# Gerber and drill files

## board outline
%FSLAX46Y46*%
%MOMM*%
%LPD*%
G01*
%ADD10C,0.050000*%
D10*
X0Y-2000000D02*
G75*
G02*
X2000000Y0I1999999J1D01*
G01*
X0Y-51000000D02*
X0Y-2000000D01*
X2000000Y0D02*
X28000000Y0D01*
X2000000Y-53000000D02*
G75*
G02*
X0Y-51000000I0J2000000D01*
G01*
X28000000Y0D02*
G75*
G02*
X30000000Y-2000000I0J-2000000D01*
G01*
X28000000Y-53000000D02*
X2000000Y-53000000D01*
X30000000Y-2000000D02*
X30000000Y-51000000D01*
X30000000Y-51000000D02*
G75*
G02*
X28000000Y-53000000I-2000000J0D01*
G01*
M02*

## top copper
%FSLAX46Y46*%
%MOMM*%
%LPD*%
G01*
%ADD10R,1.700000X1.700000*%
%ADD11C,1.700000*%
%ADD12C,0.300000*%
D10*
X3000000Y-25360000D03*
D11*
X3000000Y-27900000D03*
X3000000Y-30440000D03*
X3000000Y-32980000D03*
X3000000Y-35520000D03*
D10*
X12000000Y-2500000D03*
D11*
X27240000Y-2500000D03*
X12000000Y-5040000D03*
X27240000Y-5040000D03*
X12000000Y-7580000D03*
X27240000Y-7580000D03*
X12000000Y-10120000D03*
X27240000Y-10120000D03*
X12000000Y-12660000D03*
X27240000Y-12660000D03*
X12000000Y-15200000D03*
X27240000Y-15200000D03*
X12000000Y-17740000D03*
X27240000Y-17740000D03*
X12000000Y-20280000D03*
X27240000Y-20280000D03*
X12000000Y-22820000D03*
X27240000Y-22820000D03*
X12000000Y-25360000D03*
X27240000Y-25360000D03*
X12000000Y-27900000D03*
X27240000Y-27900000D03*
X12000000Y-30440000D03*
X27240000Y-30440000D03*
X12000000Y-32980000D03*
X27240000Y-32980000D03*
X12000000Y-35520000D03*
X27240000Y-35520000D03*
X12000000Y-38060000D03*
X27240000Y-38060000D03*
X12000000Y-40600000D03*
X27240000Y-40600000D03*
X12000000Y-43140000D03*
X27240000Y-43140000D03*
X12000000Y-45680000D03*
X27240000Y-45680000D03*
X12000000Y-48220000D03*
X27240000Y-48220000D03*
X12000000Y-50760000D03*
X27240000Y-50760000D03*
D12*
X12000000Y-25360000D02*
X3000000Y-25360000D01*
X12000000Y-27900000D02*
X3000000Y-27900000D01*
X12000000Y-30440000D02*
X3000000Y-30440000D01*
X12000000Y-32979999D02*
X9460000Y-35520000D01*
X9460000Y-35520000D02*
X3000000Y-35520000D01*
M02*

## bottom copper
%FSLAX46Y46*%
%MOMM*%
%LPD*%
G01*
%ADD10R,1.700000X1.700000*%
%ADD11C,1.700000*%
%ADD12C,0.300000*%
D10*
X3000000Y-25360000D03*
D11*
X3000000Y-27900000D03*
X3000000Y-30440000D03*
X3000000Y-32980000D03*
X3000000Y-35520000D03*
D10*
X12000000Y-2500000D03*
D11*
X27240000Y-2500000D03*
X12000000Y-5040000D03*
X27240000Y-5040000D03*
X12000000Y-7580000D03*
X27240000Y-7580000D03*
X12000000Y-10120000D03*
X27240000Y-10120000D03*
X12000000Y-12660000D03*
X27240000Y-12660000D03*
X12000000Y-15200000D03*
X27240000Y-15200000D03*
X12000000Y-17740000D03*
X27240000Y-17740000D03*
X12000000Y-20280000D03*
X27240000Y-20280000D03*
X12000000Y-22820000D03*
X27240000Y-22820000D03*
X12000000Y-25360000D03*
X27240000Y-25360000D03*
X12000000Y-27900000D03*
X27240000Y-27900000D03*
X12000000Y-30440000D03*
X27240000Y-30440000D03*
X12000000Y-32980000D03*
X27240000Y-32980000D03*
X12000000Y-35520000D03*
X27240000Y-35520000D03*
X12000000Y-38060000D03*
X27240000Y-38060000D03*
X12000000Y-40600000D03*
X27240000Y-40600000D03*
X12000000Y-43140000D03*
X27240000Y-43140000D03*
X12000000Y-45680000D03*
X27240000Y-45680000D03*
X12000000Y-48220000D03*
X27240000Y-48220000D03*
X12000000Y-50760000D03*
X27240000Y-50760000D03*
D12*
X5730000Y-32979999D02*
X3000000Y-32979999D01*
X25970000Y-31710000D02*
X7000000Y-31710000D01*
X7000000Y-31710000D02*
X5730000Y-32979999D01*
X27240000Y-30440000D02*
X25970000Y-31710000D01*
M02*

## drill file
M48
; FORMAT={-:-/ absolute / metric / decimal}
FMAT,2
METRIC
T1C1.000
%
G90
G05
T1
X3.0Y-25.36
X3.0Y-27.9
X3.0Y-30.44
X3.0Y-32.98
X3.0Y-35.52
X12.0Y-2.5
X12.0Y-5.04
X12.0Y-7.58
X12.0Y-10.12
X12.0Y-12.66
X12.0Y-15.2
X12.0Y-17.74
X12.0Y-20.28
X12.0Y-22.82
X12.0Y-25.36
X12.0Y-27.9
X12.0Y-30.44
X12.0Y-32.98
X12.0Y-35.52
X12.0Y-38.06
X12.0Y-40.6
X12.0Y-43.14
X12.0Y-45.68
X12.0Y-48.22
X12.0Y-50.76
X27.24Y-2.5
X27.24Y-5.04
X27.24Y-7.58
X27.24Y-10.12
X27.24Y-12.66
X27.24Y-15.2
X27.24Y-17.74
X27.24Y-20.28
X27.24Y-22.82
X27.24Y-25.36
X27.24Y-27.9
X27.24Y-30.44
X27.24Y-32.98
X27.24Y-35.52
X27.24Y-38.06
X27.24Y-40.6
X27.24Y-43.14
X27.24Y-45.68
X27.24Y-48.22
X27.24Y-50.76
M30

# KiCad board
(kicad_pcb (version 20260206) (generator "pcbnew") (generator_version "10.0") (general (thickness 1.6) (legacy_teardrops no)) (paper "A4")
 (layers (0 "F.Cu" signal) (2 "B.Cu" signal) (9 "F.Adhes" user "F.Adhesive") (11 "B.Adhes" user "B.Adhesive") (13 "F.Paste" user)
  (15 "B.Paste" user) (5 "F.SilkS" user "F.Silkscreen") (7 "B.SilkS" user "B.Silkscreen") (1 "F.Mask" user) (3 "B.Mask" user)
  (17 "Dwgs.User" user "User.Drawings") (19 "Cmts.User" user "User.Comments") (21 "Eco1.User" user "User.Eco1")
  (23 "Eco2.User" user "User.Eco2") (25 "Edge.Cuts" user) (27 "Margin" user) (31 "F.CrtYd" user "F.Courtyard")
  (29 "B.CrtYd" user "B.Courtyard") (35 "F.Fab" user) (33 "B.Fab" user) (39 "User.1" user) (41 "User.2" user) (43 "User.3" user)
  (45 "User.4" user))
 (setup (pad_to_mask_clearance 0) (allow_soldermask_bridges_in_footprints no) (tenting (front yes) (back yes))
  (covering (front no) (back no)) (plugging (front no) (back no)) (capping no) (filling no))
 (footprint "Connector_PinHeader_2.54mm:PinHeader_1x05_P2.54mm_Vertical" (layer "F.Cu") (at 3 25.36)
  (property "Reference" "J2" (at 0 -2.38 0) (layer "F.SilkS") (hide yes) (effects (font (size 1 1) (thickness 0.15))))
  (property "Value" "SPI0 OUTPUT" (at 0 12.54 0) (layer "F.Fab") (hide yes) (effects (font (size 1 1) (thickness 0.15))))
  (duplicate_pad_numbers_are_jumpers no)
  (pad "1" thru_hole rect (at 0 0) (size 1.7 1.7) (drill 1) (layers "*.Cu" "*.Mask") (remove_unused_layers no) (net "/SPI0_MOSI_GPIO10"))
  (pad "2" thru_hole circle (at 0 2.54) (size 1.7 1.7) (drill 1) (layers "*.Cu" "*.Mask") (remove_unused_layers no) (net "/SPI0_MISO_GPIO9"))
  (pad "3" thru_hole circle (at 0 5.08) (size 1.7 1.7) (drill 1) (layers "*.Cu" "*.Mask") (remove_unused_layers no)
   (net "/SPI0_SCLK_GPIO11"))
  (pad "4" thru_hole circle (at 0 7.62) (size 1.7 1.7) (drill 1) (layers "*.Cu" "*.Mask") (remove_unused_layers no) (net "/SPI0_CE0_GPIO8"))
  (pad "5" thru_hole circle (at 0 10.16) (size 1.7 1.7) (drill 1) (layers "*.Cu" "*.Mask") (remove_unused_layers no) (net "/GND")))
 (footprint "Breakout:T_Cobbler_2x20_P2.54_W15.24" (layer "F.Cu") (at 12 2.5)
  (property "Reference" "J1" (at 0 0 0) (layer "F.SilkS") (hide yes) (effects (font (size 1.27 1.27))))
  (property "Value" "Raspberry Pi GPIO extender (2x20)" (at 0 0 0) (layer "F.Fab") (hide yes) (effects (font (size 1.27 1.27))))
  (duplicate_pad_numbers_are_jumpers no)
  (pad "1" thru_hole rect (at 0 0) (size 1.7 1.7) (drill 1) (layers "*.Cu" "*.Mask") (remove_unused_layers no)
   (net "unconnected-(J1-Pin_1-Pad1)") (thermal_bridge_angle 45))
  (pad "2" thru_hole circle (at 15.24 0) (size 1.7 1.7) (drill 1) (layers "*.Cu" "*.Mask") (remove_unused_layers no)
   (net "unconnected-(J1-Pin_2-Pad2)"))
  (pad "3" thru_hole circle (at 0 2.54) (size 1.7 1.7) (drill 1) (layers "*.Cu" "*.Mask") (remove_unused_layers no)
   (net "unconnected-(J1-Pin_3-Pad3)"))
  (pad "4" thru_hole circle (at 15.24 2.54) (size 1.7 1.7) (drill 1) (layers "*.Cu" "*.Mask") (remove_unused_layers no)
   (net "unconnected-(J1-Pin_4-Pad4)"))
  (pad "5" thru_hole circle (at 0 5.08) (size 1.7 1.7) (drill 1) (layers "*.Cu" "*.Mask") (remove_unused_layers no)
   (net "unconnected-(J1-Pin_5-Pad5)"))
  (pad "6" thru_hole circle (at 15.24 5.08) (size 1.7 1.7) (drill 1) (layers "*.Cu" "*.Mask") (remove_unused_layers no)
   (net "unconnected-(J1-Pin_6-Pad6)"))
  (pad "7" thru_hole circle (at 0 7.62) (size 1.7 1.7) (drill 1) (layers "*.Cu" "*.Mask") (remove_unused_layers no)
   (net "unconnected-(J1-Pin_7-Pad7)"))
  (pad "8" thru_hole circle (at 15.24 7.62) (size 1.7 1.7) (drill 1) (layers "*.Cu" "*.Mask") (remove_unused_layers no)
   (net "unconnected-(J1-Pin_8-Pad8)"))
  (pad "9" thru_hole circle (at 0 10.16) (size 1.7 1.7) (drill 1) (layers "*.Cu" "*.Mask") (remove_unused_layers no)
   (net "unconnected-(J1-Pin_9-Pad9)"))
  (pad "10" thru_hole circle (at 15.24 10.16) (size 1.7 1.7) (drill 1) (layers "*.Cu" "*.Mask") (remove_unused_layers no)
   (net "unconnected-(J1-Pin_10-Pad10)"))
  (pad "11" thru_hole circle (at 0 12.7) (size 1.7 1.7) (drill 1) (layers "*.Cu" "*.Mask") (remove_unused_layers no)
   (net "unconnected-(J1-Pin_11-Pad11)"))
  (pad "12" thru_hole circle (at 15.24 12.7) (size 1.7 1.7) (drill 1) (layers "*.Cu" "*.Mask") (remove_unused_layers no)
   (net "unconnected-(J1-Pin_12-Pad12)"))
  (pad "13" thru_hole circle (at 0 15.24) (size 1.7 1.7) (drill 1) (layers "*.Cu" "*.Mask") (remove_unused_layers no)
   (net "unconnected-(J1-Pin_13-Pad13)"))
  (pad "14" thru_hole circle (at 15.24 15.24) (size 1.7 1.7) (drill 1) (layers "*.Cu" "*.Mask") (remove_unused_layers no)
   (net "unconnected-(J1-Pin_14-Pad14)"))
  (pad "15" thru_hole circle (at 0 17.78) (size 1.7 1.7) (drill 1) (layers "*.Cu" "*.Mask") (remove_unused_layers no)
   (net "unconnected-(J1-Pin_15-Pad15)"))
  (pad "16" thru_hole circle (at 15.24 17.78) (size 1.7 1.7) (drill 1) (layers "*.Cu" "*.Mask") (remove_unused_layers no)
   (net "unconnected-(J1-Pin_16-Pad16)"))
  (pad "17" thru_hole circle (at 0 20.32) (size 1.7 1.7) (drill 1) (layers "*.Cu" "*.Mask") (remove_unused_layers no)
   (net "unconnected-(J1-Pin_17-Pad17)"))
  (pad "18" thru_hole circle (at 15.24 20.32) (size 1.7 1.7) (drill 1) (layers "*.Cu" "*.Mask") (remove_unused_layers no)
   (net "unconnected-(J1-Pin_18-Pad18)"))
  (pad "19" thru_hole circle (at 0 22.86) (size 1.7 1.7) (drill 1) (layers "*.Cu" "*.Mask") (remove_unused_layers no)
   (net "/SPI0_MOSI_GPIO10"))
  (pad "20" thru_hole circle (at 15.24 22.86) (size 1.7 1.7) (drill 1) (layers "*.Cu" "*.Mask") (remove_unused_layers no)
   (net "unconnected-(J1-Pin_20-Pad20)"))
  (pad "21" thru_hole circle (at 0 25.4) (size 1.7 1.7) (drill 1) (layers "*.Cu" "*.Mask") (remove_unused_layers no)
   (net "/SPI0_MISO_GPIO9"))
  (pad "22" thru_hole circle (at 15.24 25.4) (size 1.7 1.7) (drill 1) (layers "*.Cu" "*.Mask") (remove_unused_layers no)
   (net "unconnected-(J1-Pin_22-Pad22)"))
  (pad "23" thru_hole circle (at 0 27.94) (size 1.7 1.7) (drill 1) (layers "*.Cu" "*.Mask") (remove_unused_layers no)
   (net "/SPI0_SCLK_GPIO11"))
  (pad "24" thru_hole circle (at 15.24 27.94) (size 1.7 1.7) (drill 1) (layers "*.Cu" "*.Mask") (remove_unused_layers no)
   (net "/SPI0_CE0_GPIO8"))
  (pad "25" thru_hole circle (at 0 30.48) (size 1.7 1.7) (drill 1) (layers "*.Cu" "*.Mask") (remove_unused_layers no) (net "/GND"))
  (pad "26" thru_hole circle (at 15.24 30.48) (size 1.7 1.7) (drill 1) (layers "*.Cu" "*.Mask") (remove_unused_layers no)
   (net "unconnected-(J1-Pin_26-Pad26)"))
  (pad "27" thru_hole circle (at 0 33.02) (size 1.7 1.7) (drill 1) (layers "*.Cu" "*.Mask") (remove_unused_layers no)
   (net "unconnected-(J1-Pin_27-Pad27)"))
  (pad "28" thru_hole circle (at 15.24 33.02) (size 1.7 1.7) (drill 1) (layers "*.Cu" "*.Mask") (remove_unused_layers no)
   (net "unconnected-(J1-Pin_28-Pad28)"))
  (pad "29" thru_hole circle (at 0 35.56) (size 1.7 1.7) (drill 1) (layers "*.Cu" "*.Mask") (remove_unused_layers no)
   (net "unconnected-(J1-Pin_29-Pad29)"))
  (pad "30" thru_hole circle (at 15.24 35.56) (size 1.7 1.7) (drill 1) (layers "*.Cu" "*.Mask") (remove_unused_layers no)
   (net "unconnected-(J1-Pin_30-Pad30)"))
  (pad "31" thru_hole circle (at 0 38.1) (size 1.7 1.7) (drill 1) (layers "*.Cu" "*.Mask") (remove_unused_layers no)
   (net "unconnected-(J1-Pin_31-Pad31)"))
  (pad "32" thru_hole circle (at 15.24 38.1) (size 1.7 1.7) (drill 1) (layers "*.Cu" "*.Mask") (remove_unused_layers no)
   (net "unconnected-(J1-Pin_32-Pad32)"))
  (pad "33" thru_hole circle (at 0 40.64) (size 1.7 1.7) (drill 1) (layers "*.Cu" "*.Mask") (remove_unused_layers no)
   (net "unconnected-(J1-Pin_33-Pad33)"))
  (pad "34" thru_hole circle (at 15.24 40.64) (size 1.7 1.7) (drill 1) (layers "*.Cu" "*.Mask") (remove_unused_layers no)
   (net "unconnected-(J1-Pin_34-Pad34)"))
  (pad "35" thru_hole circle (at 0 43.18) (size 1.7 1.7) (drill 1) (layers "*.Cu" "*.Mask") (remove_unused_layers no)
   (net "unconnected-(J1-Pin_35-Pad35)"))
  (pad "36" thru_hole circle (at 15.24 43.18) (size 1.7 1.7) (drill 1) (layers "*.Cu" "*.Mask") (remove_unused_layers no)
   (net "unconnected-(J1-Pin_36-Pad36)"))
  (pad "37" thru_hole circle (at 0 45.72) (size 1.7 1.7) (drill 1) (layers "*.Cu" "*.Mask") (remove_unused_layers no)
   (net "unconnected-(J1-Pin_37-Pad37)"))
  (pad "38" thru_hole circle (at 15.24 45.72) (size 1.7 1.7) (drill 1) (layers "*.Cu" "*.Mask") (remove_unused_layers no)
   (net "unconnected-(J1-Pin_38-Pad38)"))
  (pad "39" thru_hole circle (at 0 48.26) (size 1.7 1.7) (drill 1) (layers "*.Cu" "*.Mask") (remove_unused_layers no)
   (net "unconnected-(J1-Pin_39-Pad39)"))
  (pad "40" thru_hole circle (at 15.24 48.26) (size 1.7 1.7) (drill 1) (layers "*.Cu" "*.Mask") (remove_unused_layers no)
   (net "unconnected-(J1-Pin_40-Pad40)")))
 (gr_arc (start 0 2) (mid 0.585786 0.585786) (end 2 0) (stroke (width 0.05) (type default)) (layer "Edge.Cuts"))
 (gr_line (start 0 51) (end 0 2) (stroke (width 0.05) (type default)) (layer "Edge.Cuts"))
 (gr_line (start 2 0) (end 28 0) (stroke (width 0.05) (type default)) (layer "Edge.Cuts"))
 (gr_arc (start 2 53) (mid 0.585786 52.414213) (end 0 51) (stroke (width 0.05) (type default)) (layer "Edge.Cuts"))
 (gr_arc (start 28 0) (mid 29.414213 0.585786) (end 30 2) (stroke (width 0.05) (type default)) (layer "Edge.Cuts"))
 (gr_line (start 28 53) (end 2 53) (stroke (width 0.05) (type default)) (layer "Edge.Cuts"))
 (gr_line (start 30 2) (end 30 51) (stroke (width 0.05) (type default)) (layer "Edge.Cuts"))
 (gr_arc (start 30 51) (mid 29.414213 52.414213) (end 28 53) (stroke (width 0.05) (type default)) (layer "Edge.Cuts"))
 (segment (start 12 25.36) (end 3 25.36) (width 0.3) (layer "F.Cu") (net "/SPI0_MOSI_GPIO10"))
 (segment (start 12 27.9) (end 3 27.9) (width 0.3) (layer "F.Cu") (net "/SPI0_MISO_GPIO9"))
 (segment (start 12 30.44) (end 3 30.44) (width 0.3) (layer "F.Cu") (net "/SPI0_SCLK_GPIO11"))
 (segment (start 5.73 32.979999) (end 3 32.979999) (width 0.3) (layer "B.Cu") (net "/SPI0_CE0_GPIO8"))
 (segment (start 25.97 31.71) (end 7 31.71) (width 0.3) (layer "B.Cu") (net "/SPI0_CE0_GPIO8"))
 (segment (start 7 31.71) (end 5.73 32.979999) (width 0.3) (layer "B.Cu") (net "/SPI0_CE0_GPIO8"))
 (segment (start 27.24 30.44) (end 25.97 31.71) (width 0.3) (layer "B.Cu") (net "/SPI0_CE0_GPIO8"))
 (segment (start 12 32.979999) (end 9.46 35.52) (width 0.3) (layer "F.Cu") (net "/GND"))
 (segment (start 9.46 35.52) (end 3 35.52) (width 0.3) (layer "F.Cu") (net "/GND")))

